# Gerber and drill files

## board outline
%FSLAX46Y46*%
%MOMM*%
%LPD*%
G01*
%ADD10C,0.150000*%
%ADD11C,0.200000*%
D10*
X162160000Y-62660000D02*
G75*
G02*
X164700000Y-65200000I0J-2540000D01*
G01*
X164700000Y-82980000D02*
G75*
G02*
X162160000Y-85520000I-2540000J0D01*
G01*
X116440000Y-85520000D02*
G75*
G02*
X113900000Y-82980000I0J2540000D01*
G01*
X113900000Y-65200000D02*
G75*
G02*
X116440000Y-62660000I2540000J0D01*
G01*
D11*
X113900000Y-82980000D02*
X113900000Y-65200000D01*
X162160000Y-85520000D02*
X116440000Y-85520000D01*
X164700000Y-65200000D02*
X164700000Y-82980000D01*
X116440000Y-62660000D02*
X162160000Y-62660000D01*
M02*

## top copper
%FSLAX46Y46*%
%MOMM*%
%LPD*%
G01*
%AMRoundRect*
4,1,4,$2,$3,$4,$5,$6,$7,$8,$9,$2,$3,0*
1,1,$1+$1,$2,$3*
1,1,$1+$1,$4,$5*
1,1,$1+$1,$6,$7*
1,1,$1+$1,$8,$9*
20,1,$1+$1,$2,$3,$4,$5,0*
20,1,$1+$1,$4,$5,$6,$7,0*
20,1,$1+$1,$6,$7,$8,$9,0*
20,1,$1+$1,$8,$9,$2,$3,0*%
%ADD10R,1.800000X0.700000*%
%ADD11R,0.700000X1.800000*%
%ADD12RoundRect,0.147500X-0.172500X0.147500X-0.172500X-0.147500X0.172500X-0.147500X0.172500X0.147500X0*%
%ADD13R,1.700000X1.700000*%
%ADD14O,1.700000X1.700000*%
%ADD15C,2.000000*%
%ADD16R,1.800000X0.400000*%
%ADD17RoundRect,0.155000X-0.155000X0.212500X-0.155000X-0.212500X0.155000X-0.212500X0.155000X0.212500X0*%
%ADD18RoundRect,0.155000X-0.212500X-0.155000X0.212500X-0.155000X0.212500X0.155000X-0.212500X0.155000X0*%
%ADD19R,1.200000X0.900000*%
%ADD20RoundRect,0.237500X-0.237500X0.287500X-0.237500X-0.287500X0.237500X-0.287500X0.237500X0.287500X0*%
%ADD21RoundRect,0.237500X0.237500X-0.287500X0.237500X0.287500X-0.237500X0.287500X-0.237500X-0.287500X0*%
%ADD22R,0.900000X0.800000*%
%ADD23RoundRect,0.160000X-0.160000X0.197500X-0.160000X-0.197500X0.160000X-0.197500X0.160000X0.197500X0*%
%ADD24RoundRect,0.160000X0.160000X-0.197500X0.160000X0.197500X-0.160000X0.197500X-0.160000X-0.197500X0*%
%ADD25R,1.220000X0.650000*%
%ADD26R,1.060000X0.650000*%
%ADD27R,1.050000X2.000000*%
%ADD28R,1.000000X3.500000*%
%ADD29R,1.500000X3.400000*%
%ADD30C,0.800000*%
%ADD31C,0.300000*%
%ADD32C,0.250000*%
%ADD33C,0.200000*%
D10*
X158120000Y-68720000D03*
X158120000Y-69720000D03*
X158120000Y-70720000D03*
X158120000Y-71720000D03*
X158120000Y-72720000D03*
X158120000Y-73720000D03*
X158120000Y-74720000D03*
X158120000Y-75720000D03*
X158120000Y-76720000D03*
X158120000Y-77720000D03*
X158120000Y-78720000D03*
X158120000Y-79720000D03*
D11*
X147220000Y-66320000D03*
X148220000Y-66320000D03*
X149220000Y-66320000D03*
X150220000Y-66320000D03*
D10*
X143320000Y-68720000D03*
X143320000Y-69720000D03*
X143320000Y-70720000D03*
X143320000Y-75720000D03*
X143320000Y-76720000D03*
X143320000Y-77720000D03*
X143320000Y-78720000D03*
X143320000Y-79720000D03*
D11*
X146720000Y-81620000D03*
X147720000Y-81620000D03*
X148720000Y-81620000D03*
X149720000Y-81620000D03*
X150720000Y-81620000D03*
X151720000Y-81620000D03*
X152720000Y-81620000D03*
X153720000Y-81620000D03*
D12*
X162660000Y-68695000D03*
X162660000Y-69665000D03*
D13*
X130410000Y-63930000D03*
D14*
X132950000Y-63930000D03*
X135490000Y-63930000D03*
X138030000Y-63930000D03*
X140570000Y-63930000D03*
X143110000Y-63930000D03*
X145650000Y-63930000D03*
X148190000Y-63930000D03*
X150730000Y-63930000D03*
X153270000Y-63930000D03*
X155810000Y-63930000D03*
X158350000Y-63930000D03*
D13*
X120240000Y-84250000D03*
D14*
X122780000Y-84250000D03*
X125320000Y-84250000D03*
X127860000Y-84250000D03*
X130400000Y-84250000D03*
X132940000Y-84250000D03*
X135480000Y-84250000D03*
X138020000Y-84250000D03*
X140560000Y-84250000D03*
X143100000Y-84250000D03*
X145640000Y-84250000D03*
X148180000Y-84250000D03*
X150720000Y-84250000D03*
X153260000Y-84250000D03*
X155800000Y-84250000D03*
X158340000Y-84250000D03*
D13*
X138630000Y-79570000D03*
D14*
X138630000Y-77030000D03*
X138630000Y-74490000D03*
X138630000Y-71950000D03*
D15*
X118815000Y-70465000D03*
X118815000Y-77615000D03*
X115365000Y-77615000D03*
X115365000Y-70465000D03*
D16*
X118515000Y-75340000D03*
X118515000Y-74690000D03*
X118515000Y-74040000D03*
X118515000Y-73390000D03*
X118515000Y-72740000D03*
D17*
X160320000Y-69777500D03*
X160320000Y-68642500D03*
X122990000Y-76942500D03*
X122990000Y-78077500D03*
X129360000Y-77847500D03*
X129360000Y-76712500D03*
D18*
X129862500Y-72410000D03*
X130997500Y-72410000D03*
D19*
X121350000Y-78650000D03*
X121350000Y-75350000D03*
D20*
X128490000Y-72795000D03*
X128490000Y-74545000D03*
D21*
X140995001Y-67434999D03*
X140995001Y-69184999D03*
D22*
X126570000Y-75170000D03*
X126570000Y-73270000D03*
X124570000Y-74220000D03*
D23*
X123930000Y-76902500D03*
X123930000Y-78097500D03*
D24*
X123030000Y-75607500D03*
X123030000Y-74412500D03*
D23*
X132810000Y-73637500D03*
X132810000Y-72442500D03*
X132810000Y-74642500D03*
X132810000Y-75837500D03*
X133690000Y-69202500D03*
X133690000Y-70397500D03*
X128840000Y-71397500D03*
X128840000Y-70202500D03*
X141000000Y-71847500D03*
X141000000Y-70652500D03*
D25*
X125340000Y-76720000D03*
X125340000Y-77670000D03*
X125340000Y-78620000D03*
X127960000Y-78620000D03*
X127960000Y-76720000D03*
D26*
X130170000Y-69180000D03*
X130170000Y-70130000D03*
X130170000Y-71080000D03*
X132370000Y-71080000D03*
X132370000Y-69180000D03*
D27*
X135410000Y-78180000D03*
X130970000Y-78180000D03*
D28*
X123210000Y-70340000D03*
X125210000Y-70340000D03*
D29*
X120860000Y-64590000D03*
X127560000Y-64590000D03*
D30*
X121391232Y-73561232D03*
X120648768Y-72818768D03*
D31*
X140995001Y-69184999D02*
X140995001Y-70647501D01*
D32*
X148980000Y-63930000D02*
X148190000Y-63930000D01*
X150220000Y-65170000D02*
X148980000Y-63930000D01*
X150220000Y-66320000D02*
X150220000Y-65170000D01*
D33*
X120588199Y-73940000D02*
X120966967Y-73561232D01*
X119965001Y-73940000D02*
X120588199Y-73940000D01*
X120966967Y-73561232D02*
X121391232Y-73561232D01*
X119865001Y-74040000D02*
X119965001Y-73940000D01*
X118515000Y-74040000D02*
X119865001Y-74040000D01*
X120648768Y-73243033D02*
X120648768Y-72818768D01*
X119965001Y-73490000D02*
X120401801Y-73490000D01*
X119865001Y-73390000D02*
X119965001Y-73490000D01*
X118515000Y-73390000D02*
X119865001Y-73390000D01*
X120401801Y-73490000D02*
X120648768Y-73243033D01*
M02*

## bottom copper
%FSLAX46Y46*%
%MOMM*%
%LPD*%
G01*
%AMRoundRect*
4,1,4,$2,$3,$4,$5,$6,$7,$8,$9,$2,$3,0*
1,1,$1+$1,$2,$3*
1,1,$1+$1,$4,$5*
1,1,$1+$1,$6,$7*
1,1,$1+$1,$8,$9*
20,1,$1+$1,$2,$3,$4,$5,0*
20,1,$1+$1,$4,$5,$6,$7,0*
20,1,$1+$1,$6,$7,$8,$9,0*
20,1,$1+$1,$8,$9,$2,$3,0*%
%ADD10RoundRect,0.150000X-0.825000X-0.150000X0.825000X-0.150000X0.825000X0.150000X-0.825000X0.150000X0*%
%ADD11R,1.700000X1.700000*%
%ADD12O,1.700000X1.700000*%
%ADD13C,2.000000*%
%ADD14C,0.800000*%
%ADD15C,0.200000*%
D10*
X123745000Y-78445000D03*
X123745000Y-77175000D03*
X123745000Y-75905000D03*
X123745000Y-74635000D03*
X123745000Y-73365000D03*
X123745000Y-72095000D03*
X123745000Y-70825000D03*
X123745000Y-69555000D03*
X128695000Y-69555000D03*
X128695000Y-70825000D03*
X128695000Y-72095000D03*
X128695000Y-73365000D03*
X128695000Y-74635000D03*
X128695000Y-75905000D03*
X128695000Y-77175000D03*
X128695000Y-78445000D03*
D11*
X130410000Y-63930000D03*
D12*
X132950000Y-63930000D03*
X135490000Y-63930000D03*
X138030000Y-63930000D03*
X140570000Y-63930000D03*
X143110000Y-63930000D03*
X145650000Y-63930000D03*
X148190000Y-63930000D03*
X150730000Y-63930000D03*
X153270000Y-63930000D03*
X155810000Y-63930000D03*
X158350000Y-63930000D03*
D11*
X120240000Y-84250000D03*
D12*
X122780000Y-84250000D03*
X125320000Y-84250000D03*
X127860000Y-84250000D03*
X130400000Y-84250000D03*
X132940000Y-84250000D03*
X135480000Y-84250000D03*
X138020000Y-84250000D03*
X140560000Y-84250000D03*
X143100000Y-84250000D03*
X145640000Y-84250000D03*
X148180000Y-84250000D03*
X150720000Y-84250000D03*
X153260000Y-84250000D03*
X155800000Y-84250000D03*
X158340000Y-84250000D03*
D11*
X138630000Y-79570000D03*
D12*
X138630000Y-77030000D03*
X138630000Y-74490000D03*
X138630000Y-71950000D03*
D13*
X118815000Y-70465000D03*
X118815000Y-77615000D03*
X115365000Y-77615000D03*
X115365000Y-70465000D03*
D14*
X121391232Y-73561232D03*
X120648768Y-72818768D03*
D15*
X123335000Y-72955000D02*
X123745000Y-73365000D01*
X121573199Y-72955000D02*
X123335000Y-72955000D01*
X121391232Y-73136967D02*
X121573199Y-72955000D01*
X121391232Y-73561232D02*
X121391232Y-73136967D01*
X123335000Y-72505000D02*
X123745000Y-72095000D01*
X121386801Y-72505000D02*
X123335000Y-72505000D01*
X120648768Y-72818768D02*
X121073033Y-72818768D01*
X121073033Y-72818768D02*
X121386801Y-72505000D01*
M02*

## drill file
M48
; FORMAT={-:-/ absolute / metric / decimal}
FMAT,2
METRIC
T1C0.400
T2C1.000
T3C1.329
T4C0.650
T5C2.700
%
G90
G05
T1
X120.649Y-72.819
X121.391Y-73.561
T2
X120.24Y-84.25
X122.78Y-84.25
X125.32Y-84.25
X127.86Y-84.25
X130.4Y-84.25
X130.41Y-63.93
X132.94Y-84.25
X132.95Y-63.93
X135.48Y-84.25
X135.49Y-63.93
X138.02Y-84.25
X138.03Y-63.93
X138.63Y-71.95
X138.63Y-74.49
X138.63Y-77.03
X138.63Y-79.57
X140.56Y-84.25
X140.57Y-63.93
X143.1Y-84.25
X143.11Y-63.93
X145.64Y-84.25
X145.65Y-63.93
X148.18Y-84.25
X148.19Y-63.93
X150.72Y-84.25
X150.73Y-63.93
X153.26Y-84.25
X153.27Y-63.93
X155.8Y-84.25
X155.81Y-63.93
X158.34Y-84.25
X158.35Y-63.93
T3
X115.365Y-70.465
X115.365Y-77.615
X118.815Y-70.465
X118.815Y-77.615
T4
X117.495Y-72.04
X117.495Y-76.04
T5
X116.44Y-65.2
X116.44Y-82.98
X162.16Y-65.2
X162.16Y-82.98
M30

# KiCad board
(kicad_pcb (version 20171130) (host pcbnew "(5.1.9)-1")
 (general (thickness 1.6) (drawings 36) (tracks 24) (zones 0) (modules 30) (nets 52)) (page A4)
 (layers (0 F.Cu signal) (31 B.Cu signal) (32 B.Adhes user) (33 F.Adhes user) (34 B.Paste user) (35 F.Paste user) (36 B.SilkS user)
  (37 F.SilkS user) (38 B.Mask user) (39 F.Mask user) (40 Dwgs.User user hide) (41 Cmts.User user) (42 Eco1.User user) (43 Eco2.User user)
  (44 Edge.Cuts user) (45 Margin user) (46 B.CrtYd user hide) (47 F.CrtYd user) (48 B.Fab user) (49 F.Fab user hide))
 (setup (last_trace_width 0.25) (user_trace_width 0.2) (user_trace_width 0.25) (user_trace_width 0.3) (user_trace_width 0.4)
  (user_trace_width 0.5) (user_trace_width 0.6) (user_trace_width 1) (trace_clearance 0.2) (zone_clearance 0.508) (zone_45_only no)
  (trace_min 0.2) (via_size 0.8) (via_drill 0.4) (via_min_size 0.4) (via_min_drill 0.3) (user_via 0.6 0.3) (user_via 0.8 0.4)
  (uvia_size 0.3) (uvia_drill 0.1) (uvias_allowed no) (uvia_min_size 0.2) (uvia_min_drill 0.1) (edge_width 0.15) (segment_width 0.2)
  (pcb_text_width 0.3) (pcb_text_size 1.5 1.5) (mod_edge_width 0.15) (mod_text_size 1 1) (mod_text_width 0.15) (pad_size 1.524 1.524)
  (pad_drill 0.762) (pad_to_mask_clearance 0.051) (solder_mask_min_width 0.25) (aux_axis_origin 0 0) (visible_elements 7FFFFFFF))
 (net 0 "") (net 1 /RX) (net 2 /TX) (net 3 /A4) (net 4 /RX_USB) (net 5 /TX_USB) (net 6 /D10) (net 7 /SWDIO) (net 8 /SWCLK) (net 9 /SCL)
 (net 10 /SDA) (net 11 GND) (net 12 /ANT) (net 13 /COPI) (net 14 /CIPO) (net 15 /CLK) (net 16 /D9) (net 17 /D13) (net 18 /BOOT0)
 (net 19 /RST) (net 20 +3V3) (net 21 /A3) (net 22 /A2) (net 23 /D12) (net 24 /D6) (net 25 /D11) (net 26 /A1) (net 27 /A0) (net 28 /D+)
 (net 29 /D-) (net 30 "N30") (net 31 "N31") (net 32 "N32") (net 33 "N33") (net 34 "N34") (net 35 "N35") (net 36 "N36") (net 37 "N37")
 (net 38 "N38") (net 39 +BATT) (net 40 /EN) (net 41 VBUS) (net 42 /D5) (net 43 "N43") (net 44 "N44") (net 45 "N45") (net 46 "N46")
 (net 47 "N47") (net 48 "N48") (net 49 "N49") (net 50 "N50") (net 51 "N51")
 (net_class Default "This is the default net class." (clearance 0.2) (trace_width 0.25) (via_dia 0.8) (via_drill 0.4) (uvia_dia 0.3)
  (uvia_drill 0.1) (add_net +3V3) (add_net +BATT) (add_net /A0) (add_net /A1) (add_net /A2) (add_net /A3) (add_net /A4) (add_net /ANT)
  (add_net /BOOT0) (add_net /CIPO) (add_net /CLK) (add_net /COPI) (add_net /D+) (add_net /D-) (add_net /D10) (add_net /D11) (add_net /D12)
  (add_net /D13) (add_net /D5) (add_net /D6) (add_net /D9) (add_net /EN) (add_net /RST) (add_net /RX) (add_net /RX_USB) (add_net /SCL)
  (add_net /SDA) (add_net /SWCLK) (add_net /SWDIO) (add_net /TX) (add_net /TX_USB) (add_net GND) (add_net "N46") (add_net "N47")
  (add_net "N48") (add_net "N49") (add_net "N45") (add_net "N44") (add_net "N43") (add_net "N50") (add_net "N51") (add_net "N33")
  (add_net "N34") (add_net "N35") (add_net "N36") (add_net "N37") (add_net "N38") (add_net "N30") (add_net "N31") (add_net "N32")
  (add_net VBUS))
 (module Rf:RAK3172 (layer F.Cu) (at 158.22 66.22 270)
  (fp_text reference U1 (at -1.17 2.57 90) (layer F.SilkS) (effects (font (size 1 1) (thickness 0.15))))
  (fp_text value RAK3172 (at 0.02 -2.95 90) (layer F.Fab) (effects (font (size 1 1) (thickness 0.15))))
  (pad 1 smd rect (at 2.5 0.1 270) (size 0.7 1.8) (layers F.Cu F.Paste F.Mask) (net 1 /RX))
  (pad 2 smd rect (at 3.5 0.1 270) (size 0.7 1.8) (layers F.Cu F.Paste F.Mask) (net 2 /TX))
  (pad 3 smd rect (at 4.5 0.1 270) (size 0.7 1.8) (layers F.Cu F.Paste F.Mask) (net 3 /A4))
  (pad 4 smd rect (at 5.5 0.1 270) (size 0.7 1.8) (layers F.Cu F.Paste F.Mask) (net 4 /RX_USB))
  (pad 5 smd rect (at 6.5 0.1 270) (size 0.7 1.8) (layers F.Cu F.Paste F.Mask) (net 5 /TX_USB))
  (pad 6 smd rect (at 7.5 0.1 270) (size 0.7 1.8) (layers F.Cu F.Paste F.Mask) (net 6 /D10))
  (pad 7 smd rect (at 8.5 0.1 270) (size 0.7 1.8) (layers F.Cu F.Paste F.Mask) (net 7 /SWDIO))
  (pad 8 smd rect (at 9.5 0.1 270) (size 0.7 1.8) (layers F.Cu F.Paste F.Mask) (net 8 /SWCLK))
  (pad 9 smd rect (at 10.5 0.1 270) (size 0.7 1.8) (layers F.Cu F.Paste F.Mask) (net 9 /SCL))
  (pad 10 smd rect (at 11.5 0.1 270) (size 0.7 1.8) (layers F.Cu F.Paste F.Mask) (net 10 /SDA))
  (pad 11 smd rect (at 12.5 0.1 270) (size 0.7 1.8) (layers F.Cu F.Paste F.Mask) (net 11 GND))
  (pad 12 smd rect (at 13.5 0.1 270) (size 0.7 1.8) (layers F.Cu F.Paste F.Mask) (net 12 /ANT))
  (pad 13 smd rect (at 0.1 11) (size 0.7 1.8) (layers F.Cu F.Paste F.Mask) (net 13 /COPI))
  (pad 14 smd rect (at 0.1 10) (size 0.7 1.8) (layers F.Cu F.Paste F.Mask) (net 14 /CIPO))
  (pad 15 smd rect (at 0.1 9) (size 0.7 1.8) (layers F.Cu F.Paste F.Mask) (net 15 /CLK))
  (pad 16 smd rect (at 0.1 8) (size 0.7 1.8) (layers F.Cu F.Paste F.Mask) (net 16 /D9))
  (pad 17 smd rect (at 2.5 14.9 270) (size 0.7 1.8) (layers F.Cu F.Paste F.Mask) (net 11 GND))
  (pad 18 smd rect (at 3.5 14.9 270) (size 0.7 1.8) (layers F.Cu F.Paste F.Mask) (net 11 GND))
  (pad 19 smd rect (at 4.5 14.9 270) (size 0.7 1.8) (layers F.Cu F.Paste F.Mask) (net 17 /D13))
  (pad 20 smd rect (at 9.5 14.9 270) (size 0.7 1.8) (layers F.Cu F.Paste F.Mask))
  (pad 21 smd rect (at 10.5 14.9 270) (size 0.7 1.8) (layers F.Cu F.Paste F.Mask) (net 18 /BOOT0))
  (pad 22 smd rect (at 11.5 14.9 270) (size 0.7 1.8) (layers F.Cu F.Paste F.Mask) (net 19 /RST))
  (pad 23 smd rect (at 12.5 14.9 270) (size 0.7 1.8) (layers F.Cu F.Paste F.Mask) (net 11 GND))
  (pad 24 smd rect (at 13.5 14.9 270) (size 0.7 1.8) (layers F.Cu F.Paste F.Mask) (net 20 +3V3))
  (pad 25 smd rect (at 15.4 11.5) (size 0.7 1.8) (layers F.Cu F.Paste F.Mask) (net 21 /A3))
  (pad 26 smd rect (at 15.4 10.5) (size 0.7 1.8) (layers F.Cu F.Paste F.Mask) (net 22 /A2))
  (pad 27 smd rect (at 15.4 9.5) (size 0.7 1.8) (layers F.Cu F.Paste F.Mask) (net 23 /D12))
  (pad 28 smd rect (at 15.4 8.5) (size 0.7 1.8) (layers F.Cu F.Paste F.Mask) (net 11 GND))
  (pad 29 smd rect (at 15.4 7.5) (size 0.7 1.8) (layers F.Cu F.Paste F.Mask) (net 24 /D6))
  (pad 30 smd rect (at 15.4 6.5) (size 0.7 1.8) (layers F.Cu F.Paste F.Mask) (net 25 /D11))
  (pad 31 smd rect (at 15.4 5.5) (size 0.7 1.8) (layers F.Cu F.Paste F.Mask) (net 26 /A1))
  (pad 32 smd rect (at 15.4 4.5) (size 0.7 1.8) (layers F.Cu F.Paste F.Mask) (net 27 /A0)))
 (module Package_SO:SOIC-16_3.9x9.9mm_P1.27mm (layer B.Cu) (at 126.22 74)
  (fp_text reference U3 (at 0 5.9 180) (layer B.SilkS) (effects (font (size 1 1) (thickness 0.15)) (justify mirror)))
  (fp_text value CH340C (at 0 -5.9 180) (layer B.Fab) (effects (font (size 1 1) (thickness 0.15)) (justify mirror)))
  (pad 1 smd roundrect (at -2.475 4.445) (size 1.95 0.6) (layers B.Cu B.Paste B.Mask) (roundrect_rratio 0.25) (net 11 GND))
  (pad 2 smd roundrect (at -2.475 3.175) (size 1.95 0.6) (layers B.Cu B.Paste B.Mask) (roundrect_rratio 0.25) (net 5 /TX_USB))
  (pad 3 smd roundrect (at -2.475 1.905) (size 1.95 0.6) (layers B.Cu B.Paste B.Mask) (roundrect_rratio 0.25) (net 4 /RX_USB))
  (pad 4 smd roundrect (at -2.475 0.635) (size 1.95 0.6) (layers B.Cu B.Paste B.Mask) (roundrect_rratio 0.25) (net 20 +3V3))
  (pad 5 smd roundrect (at -2.475 -0.635) (size 1.95 0.6) (layers B.Cu B.Paste B.Mask) (roundrect_rratio 0.25) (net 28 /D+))
  (pad 6 smd roundrect (at -2.475 -1.905) (size 1.95 0.6) (layers B.Cu B.Paste B.Mask) (roundrect_rratio 0.25) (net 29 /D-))
  (pad 7 smd roundrect (at -2.475 -3.175) (size 1.95 0.6) (layers B.Cu B.Paste B.Mask) (roundrect_rratio 0.25) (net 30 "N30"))
  (pad 8 smd roundrect (at -2.475 -4.445) (size 1.95 0.6) (layers B.Cu B.Paste B.Mask) (roundrect_rratio 0.25) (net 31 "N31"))
  (pad 9 smd roundrect (at 2.475 -4.445) (size 1.95 0.6) (layers B.Cu B.Paste B.Mask) (roundrect_rratio 0.25) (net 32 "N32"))
  (pad 10 smd roundrect (at 2.475 -3.175) (size 1.95 0.6) (layers B.Cu B.Paste B.Mask) (roundrect_rratio 0.25) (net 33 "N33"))
  (pad 11 smd roundrect (at 2.475 -1.905) (size 1.95 0.6) (layers B.Cu B.Paste B.Mask) (roundrect_rratio 0.25) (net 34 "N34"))
  (pad 12 smd roundrect (at 2.475 -0.635) (size 1.95 0.6) (layers B.Cu B.Paste B.Mask) (roundrect_rratio 0.25) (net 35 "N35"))
  (pad 13 smd roundrect (at 2.475 0.635) (size 1.95 0.6) (layers B.Cu B.Paste B.Mask) (roundrect_rratio 0.25) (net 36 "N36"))
  (pad 14 smd roundrect (at 2.475 1.905) (size 1.95 0.6) (layers B.Cu B.Paste B.Mask) (roundrect_rratio 0.25) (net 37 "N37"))
  (pad 15 smd roundrect (at 2.475 3.175) (size 1.95 0.6) (layers B.Cu B.Paste B.Mask) (roundrect_rratio 0.25) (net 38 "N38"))
  (pad 16 smd roundrect (at 2.475 4.445) (size 1.95 0.6) (layers B.Cu B.Paste B.Mask) (roundrect_rratio 0.25) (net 20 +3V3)))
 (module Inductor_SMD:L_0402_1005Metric (layer F.Cu) (at 162.66 69.18 270)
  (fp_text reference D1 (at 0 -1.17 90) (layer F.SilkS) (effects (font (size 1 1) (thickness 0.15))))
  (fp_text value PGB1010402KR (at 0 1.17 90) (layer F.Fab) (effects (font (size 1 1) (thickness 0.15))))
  (pad 1 smd roundrect (at -0.485 0 270) (size 0.59 0.64) (layers F.Cu F.Paste F.Mask) (roundrect_rratio 0.25) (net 12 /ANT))
  (pad 2 smd roundrect (at 0.485 0 270) (size 0.59 0.64) (layers F.Cu F.Paste F.Mask) (roundrect_rratio 0.25) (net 11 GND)))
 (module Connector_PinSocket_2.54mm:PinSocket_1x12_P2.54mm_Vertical (layer F.Cu) (at 130.41 63.93 90)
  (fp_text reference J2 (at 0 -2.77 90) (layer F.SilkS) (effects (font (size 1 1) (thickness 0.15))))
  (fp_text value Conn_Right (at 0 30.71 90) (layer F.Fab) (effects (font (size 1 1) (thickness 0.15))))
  (pad 1 thru_hole rect (at 0 0 90) (size 1.7 1.7) (drill 1) (layers *.Cu *.Mask) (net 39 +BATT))
  (pad 2 thru_hole oval (at 0 2.54 90) (size 1.7 1.7) (drill 1) (layers *.Cu *.Mask) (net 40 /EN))
  (pad 3 thru_hole oval (at 0 5.08 90) (size 1.7 1.7) (drill 1) (layers *.Cu *.Mask) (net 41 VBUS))
  (pad 4 thru_hole oval (at 0 7.62 90) (size 1.7 1.7) (drill 1) (layers *.Cu *.Mask) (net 17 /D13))
  (pad 5 thru_hole oval (at 0 10.16 90) (size 1.7 1.7) (drill 1) (layers *.Cu *.Mask) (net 23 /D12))
  (pad 6 thru_hole oval (at 0 12.7 90) (size 1.7 1.7) (drill 1) (layers *.Cu *.Mask) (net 25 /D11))
  (pad 7 thru_hole oval (at 0 15.24 90) (size 1.7 1.7) (drill 1) (layers *.Cu *.Mask) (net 6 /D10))
  (pad 8 thru_hole oval (at 0 17.78 90) (size 1.7 1.7) (drill 1) (layers *.Cu *.Mask) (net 16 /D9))
  (pad 9 thru_hole oval (at 0 20.32 90) (size 1.7 1.7) (drill 1) (layers *.Cu *.Mask) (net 24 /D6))
  (pad 10 thru_hole oval (at 0 22.86 90) (size 1.7 1.7) (drill 1) (layers *.Cu *.Mask) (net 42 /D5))
  (pad 11 thru_hole oval (at 0 25.4 90) (size 1.7 1.7) (drill 1) (layers *.Cu *.Mask) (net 9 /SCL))
  (pad 12 thru_hole oval (at 0 27.94 90) (size 1.7 1.7) (drill 1) (layers *.Cu *.Mask) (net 10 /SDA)))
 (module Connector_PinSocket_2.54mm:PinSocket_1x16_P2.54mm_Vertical (layer F.Cu) (at 120.24 84.25 90)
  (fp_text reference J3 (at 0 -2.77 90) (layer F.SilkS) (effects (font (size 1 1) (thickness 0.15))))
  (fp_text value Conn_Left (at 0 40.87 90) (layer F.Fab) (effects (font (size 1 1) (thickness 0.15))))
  (pad 1 thru_hole rect (at 0 0 90) (size 1.7 1.7) (drill 1) (layers *.Cu *.Mask) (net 19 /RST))
  (pad 2 thru_hole oval (at 0 2.54 90) (size 1.7 1.7) (drill 1) (layers *.Cu *.Mask) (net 20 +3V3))
  (pad 3 thru_hole oval (at 0 5.08 90) (size 1.7 1.7) (drill 1) (layers *.Cu *.Mask) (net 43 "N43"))
  (pad 4 thru_hole oval (at 0 7.62 90) (size 1.7 1.7) (drill 1) (layers *.Cu *.Mask) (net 11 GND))
  (pad 5 thru_hole oval (at 0 10.16 90) (size 1.7 1.7) (drill 1) (layers *.Cu *.Mask) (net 27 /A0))
  (pad 6 thru_hole oval (at 0 12.7 90) (size 1.7 1.7) (drill 1) (layers *.Cu *.Mask) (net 26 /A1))
  (pad 7 thru_hole oval (at 0 15.24 90) (size 1.7 1.7) (drill 1) (layers *.Cu *.Mask) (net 22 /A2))
  (pad 8 thru_hole oval (at 0 17.78 90) (size 1.7 1.7) (drill 1) (layers *.Cu *.Mask) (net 21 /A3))
  (pad 9 thru_hole oval (at 0 20.32 90) (size 1.7 1.7) (drill 1) (layers *.Cu *.Mask) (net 3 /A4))
  (pad 10 thru_hole oval (at 0 22.86 90) (size 1.7 1.7) (drill 1) (layers *.Cu *.Mask) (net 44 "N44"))
  (pad 11 thru_hole oval (at 0 25.4 90) (size 1.7 1.7) (drill 1) (layers *.Cu *.Mask) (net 15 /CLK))
  (pad 12 thru_hole oval (at 0 27.94 90) (size 1.7 1.7) (drill 1) (layers *.Cu *.Mask) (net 13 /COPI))
  (pad 13 thru_hole oval (at 0 30.48 90) (size 1.7 1.7) (drill 1) (layers *.Cu *.Mask) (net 14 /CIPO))
  (pad 14 thru_hole oval (at 0 33.02 90) (size 1.7 1.7) (drill 1) (layers *.Cu *.Mask) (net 1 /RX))
  (pad 15 thru_hole oval (at 0 35.56 90) (size 1.7 1.7) (drill 1) (layers *.Cu *.Mask) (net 2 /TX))
  (pad 16 thru_hole oval (at 0 38.1 90) (size 1.7 1.7) (drill 1) (layers *.Cu *.Mask) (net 18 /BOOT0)))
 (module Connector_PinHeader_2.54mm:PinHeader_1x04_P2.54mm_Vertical (layer F.Cu) (at 138.63 79.57 180)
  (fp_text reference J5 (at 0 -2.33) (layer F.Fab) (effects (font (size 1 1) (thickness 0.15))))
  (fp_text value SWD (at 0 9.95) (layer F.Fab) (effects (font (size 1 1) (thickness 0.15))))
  (pad 1 thru_hole rect (at 0 0 180) (size 1.7 1.7) (drill 1) (layers *.Cu *.Mask) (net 20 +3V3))
  (pad 2 thru_hole oval (at 0 2.54 180) (size 1.7 1.7) (drill 1) (layers *.Cu *.Mask) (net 7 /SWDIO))
  (pad 3 thru_hole oval (at 0 5.08 180) (size 1.7 1.7) (drill 1) (layers *.Cu *.Mask) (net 8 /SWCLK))
  (pad 4 thru_hole oval (at 0 7.62 180) (size 1.7 1.7) (drill 1) (layers *.Cu *.Mask) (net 11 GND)))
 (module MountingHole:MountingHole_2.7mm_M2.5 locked (layer F.Cu) (at 162.16 65.2)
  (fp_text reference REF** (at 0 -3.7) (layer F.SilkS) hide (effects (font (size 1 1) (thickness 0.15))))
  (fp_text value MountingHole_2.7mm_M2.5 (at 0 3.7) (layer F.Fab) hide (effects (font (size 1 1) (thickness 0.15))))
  (pad 1 np_thru_hole circle (at 0 0) (size 2.7 2.7) (drill 2.7) (layers *.Cu *.Mask)))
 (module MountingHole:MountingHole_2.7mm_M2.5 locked (layer F.Cu) (at 162.16 82.98)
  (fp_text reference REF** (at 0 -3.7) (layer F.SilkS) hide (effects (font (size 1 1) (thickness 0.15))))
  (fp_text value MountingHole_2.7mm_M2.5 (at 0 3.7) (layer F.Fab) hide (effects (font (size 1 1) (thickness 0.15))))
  (pad 1 np_thru_hole circle (at 0 0) (size 2.7 2.7) (drill 2.7) (layers *.Cu *.Mask)))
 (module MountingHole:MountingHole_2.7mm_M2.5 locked (layer F.Cu) (at 116.44 82.98)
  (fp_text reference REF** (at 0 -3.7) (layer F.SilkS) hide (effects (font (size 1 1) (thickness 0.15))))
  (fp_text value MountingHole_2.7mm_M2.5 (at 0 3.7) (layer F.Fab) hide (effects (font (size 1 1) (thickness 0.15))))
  (pad 1 np_thru_hole circle (at 0 0) (size 2.7 2.7) (drill 2.7) (layers *.Cu *.Mask)))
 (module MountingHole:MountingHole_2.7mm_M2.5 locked (layer F.Cu) (at 116.44 65.2)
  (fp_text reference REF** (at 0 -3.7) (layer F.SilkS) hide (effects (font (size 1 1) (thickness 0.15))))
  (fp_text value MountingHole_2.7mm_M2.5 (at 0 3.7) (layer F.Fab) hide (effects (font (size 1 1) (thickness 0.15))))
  (pad 1 np_thru_hole circle (at 0 0) (size 2.7 2.7) (drill 2.7) (layers *.Cu *.Mask)))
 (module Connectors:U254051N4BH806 (layer F.Cu) (at 116.33 74.04 270)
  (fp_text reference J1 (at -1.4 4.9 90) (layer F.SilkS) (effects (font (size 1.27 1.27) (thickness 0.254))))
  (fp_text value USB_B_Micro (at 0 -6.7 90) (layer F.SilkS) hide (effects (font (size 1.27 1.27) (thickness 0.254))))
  (pad MH6 np_thru_hole circle (at 2 -1.165 270) (size 0.65 0) (drill 0.65) (layers *.Cu *.Mask))
  (pad MH5 np_thru_hole circle (at -2 -1.165 270) (size 0.65 0) (drill 0.65) (layers *.Cu *.Mask))
  (pad 6 thru_hole circle (at -3.575 -2.485 270) (size 2 2) (drill 1.3285) (layers *.Cu *.Mask) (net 11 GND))
  (pad 6 thru_hole circle (at 3.575 -2.485 270) (size 2 2) (drill 1.3285) (layers *.Cu *.Mask) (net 11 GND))
  (pad 6 thru_hole circle (at 3.575 0.965 270) (size 2 2) (drill 1.3285) (layers *.Cu *.Mask) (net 11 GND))
  (pad 6 thru_hole circle (at -3.575 0.965 270) (size 2 2) (drill 1.3285) (layers *.Cu *.Mask) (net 11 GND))
  (pad 5 smd rect (at 1.3 -2.185 270) (size 0.4 1.8) (layers F.Cu F.Paste F.Mask) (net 11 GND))
  (pad 4 smd rect (at 0.65 -2.185 270) (size 0.4 1.8) (layers F.Cu F.Paste F.Mask) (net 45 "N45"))
  (pad 3 smd rect (at 0 -2.185 270) (size 0.4 1.8) (layers F.Cu F.Paste F.Mask) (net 28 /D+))
  (pad 2 smd rect (at -0.65 -2.185 270) (size 0.4 1.8) (layers F.Cu F.Paste F.Mask) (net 29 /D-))
  (pad 1 smd rect (at -1.3 -2.185 270) (size 0.4 1.8) (layers F.Cu F.Paste F.Mask) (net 41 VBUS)))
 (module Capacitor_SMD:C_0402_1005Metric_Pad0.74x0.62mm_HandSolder (layer F.Cu) (at 160.32 69.21 270)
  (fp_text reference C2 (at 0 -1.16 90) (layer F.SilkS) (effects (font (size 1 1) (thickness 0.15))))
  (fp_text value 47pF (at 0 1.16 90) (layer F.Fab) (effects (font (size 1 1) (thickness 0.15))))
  (pad 2 smd roundrect (at 0.5675 0 270) (size 0.735 0.62) (layers F.Cu F.Paste F.Mask) (roundrect_rratio 0.25) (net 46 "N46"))
  (pad 1 smd roundrect (at -0.5675 0 270) (size 0.735 0.62) (layers F.Cu F.Paste F.Mask) (roundrect_rratio 0.25) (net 12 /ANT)))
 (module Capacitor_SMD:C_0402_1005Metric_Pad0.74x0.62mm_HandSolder (layer F.Cu) (at 122.99 77.51 270)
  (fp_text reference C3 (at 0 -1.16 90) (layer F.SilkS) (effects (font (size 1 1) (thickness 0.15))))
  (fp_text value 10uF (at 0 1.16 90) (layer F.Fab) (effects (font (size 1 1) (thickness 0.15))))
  (pad 1 smd roundrect (at -0.5675 0 270) (size 0.735 0.62) (layers F.Cu F.Paste F.Mask) (roundrect_rratio 0.25) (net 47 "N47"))
  (pad 2 smd roundrect (at 0.5675 0 270) (size 0.735 0.62) (layers F.Cu F.Paste F.Mask) (roundrect_rratio 0.25) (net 11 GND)))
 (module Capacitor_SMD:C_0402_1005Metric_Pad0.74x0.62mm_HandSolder (layer F.Cu) (at 129.36 77.28 270)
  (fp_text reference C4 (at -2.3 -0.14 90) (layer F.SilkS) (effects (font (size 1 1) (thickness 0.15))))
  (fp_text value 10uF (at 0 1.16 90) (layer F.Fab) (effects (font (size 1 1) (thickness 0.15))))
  (pad 2 smd roundrect (at 0.5675 0 270) (size 0.735 0.62) (layers F.Cu F.Paste F.Mask) (roundrect_rratio 0.25) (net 11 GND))
  (pad 1 smd roundrect (at -0.5675 0 270) (size 0.735 0.62) (layers F.Cu F.Paste F.Mask) (roundrect_rratio 0.25) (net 20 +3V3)))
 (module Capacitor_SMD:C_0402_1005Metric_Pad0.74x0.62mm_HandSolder (layer F.Cu) (at 130.43 72.41)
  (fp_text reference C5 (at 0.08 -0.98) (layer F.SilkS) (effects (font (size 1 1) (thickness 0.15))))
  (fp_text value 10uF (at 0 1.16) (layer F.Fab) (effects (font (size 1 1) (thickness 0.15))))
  (pad 1 smd roundrect (at -0.5675 0) (size 0.735 0.62) (layers F.Cu F.Paste F.Mask) (roundrect_rratio 0.25) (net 39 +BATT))
  (pad 2 smd roundrect (at 0.5675 0) (size 0.735 0.62) (layers F.Cu F.Paste F.Mask) (roundrect_rratio 0.25) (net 11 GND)))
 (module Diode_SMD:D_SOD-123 (layer F.Cu) (at 121.35 77 90)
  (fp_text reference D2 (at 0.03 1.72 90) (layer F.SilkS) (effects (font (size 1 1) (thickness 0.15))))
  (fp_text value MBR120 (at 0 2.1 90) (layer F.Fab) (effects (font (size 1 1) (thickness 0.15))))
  (pad 1 smd rect (at -1.65 0 90) (size 0.9 1.2) (layers F.Cu F.Paste F.Mask) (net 47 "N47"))
  (pad 2 smd rect (at 1.65 0 90) (size 0.9 1.2) (layers F.Cu F.Paste F.Mask) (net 41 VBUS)))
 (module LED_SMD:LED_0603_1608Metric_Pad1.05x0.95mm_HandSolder (layer F.Cu) (at 128.49 73.67 270)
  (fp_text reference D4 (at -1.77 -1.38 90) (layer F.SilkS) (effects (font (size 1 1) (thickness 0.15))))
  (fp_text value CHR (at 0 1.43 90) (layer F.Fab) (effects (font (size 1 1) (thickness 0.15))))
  (pad 1 smd roundrect (at -0.875 0 270) (size 1.05 0.95) (layers F.Cu F.Paste F.Mask) (roundrect_rratio 0.25) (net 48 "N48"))
  (pad 2 smd roundrect (at 0.875 0 270) (size 1.05 0.95) (layers F.Cu F.Paste F.Mask) (roundrect_rratio 0.25) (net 41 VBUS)))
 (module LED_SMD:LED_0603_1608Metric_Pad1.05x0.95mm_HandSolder (layer F.Cu) (at 140.995001 68.309999 90)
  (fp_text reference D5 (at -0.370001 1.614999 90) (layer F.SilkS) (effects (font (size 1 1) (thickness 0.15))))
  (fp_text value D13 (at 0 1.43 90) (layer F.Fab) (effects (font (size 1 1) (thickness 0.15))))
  (pad 2 smd roundrect (at 0.875 0 90) (size 1.05 0.95) (layers F.Cu F.Paste F.Mask) (roundrect_rratio 0.25) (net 17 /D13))
  (pad 1 smd roundrect (at -0.875 0 90) (size 1.05 0.95) (layers F.Cu F.Paste F.Mask) (roundrect_rratio 0.25) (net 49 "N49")))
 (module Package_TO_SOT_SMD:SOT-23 (layer F.Cu) (at 125.57 74.22 180)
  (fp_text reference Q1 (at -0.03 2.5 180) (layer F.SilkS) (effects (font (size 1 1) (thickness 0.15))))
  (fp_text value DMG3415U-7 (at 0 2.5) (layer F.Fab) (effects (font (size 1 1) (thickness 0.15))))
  (pad 1 smd rect (at -1 -0.95 180) (size 0.9 0.8) (layers F.Cu F.Paste F.Mask) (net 41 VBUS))
  (pad 2 smd rect (at -1 0.95 180) (size 0.9 0.8) (layers F.Cu F.Paste F.Mask) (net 47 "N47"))
  (pad 3 smd rect (at 1 0 180) (size 0.9 0.8) (layers F.Cu F.Paste F.Mask) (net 39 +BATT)))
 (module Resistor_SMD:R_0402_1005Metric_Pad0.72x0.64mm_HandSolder (layer F.Cu) (at 123.93 77.5 270)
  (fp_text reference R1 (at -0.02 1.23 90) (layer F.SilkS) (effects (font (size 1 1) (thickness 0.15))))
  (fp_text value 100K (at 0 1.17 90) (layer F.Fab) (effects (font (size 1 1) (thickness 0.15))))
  (pad 1 smd roundrect (at -0.5975 0 270) (size 0.715 0.64) (layers F.Cu F.Paste F.Mask) (roundrect_rratio 0.25) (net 47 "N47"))
  (pad 2 smd roundrect (at 0.5975 0 270) (size 0.715 0.64) (layers F.Cu F.Paste F.Mask) (roundrect_rratio 0.25) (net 40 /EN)))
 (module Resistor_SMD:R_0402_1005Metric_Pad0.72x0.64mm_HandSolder (layer F.Cu) (at 123.03 75.01 90)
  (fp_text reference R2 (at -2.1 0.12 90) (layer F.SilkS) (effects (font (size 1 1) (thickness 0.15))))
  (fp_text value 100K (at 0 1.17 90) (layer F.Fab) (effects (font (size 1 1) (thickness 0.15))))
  (pad 1 smd roundrect (at -0.5975 0 90) (size 0.715 0.64) (layers F.Cu F.Paste F.Mask) (roundrect_rratio 0.25) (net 41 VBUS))
  (pad 2 smd roundrect (at 0.5975 0 90) (size 0.715 0.64) (layers F.Cu F.Paste F.Mask) (roundrect_rratio 0.25) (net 11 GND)))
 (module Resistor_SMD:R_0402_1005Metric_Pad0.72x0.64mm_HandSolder (layer F.Cu) (at 132.81 73.04 270)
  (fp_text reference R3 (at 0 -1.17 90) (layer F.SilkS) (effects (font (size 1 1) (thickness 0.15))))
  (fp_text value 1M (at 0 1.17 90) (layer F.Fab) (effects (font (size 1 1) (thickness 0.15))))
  (pad 2 smd roundrect (at 0.5975 0 270) (size 0.715 0.64) (layers F.Cu F.Paste F.Mask) (roundrect_rratio 0.25) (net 27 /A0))
  (pad 1 smd roundrect (at -0.5975 0 270) (size 0.715 0.64) (layers F.Cu F.Paste F.Mask) (roundrect_rratio 0.25) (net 39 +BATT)))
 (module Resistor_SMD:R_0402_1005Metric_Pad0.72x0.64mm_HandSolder (layer F.Cu) (at 132.81 75.24 270)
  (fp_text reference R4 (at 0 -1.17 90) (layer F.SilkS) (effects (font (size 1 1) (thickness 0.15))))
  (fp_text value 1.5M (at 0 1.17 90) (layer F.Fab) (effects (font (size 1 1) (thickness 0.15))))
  (pad 1 smd roundrect (at -0.5975 0 270) (size 0.715 0.64) (layers F.Cu F.Paste F.Mask) (roundrect_rratio 0.25) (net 27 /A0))
  (pad 2 smd roundrect (at 0.5975 0 270) (size 0.715 0.64) (layers F.Cu F.Paste F.Mask) (roundrect_rratio 0.25) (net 11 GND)))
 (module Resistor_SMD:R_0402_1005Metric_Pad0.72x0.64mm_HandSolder (layer F.Cu) (at 133.69 69.8 270)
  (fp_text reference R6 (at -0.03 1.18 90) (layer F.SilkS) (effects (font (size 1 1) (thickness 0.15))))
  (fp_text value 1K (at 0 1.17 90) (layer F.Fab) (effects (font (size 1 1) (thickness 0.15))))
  (pad 1 smd roundrect (at -0.5975 0 270) (size 0.715 0.64) (layers F.Cu F.Paste F.Mask) (roundrect_rratio 0.25) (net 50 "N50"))
  (pad 2 smd roundrect (at 0.5975 0 270) (size 0.715 0.64) (layers F.Cu F.Paste F.Mask) (roundrect_rratio 0.25) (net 11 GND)))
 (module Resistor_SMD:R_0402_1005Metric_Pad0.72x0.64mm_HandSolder (layer F.Cu) (at 128.84 70.8 270)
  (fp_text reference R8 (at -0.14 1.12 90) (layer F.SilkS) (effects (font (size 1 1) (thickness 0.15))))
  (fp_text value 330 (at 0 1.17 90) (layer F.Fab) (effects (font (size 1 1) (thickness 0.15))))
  (pad 2 smd roundrect (at 0.5975 0 270) (size 0.715 0.64) (layers F.Cu F.Paste F.Mask) (roundrect_rratio 0.25) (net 48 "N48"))
  (pad 1 smd roundrect (at -0.5975 0 270) (size 0.715 0.64) (layers F.Cu F.Paste F.Mask) (roundrect_rratio 0.25) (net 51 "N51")))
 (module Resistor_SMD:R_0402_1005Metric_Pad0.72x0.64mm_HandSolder (layer F.Cu) (at 141 71.25 270)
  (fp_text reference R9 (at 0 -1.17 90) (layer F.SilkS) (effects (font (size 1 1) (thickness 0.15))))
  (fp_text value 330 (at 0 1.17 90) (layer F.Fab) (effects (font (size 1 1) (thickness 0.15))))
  (pad 2 smd roundrect (at 0.5975 0 270) (size 0.715 0.64) (layers F.Cu F.Paste F.Mask) (roundrect_rratio 0.25) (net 11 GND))
  (pad 1 smd roundrect (at -0.5975 0 270) (size 0.715 0.64) (layers F.Cu F.Paste F.Mask) (roundrect_rratio 0.25) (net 49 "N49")))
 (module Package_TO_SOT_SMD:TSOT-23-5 (layer F.Cu) (at 126.65 77.67)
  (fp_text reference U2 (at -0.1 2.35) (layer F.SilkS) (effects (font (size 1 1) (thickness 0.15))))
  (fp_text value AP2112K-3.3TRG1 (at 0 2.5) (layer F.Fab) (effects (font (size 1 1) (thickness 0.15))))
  (pad 1 smd rect (at -1.31 -0.95) (size 1.22 0.65) (layers F.Cu F.Paste F.Mask) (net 47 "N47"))
  (pad 2 smd rect (at -1.31 0) (size 1.22 0.65) (layers F.Cu F.Paste F.Mask) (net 11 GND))
  (pad 3 smd rect (at -1.31 0.95) (size 1.22 0.65) (layers F.Cu F.Paste F.Mask) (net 40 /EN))
  (pad 4 smd rect (at 1.31 0.95) (size 1.22 0.65) (layers F.Cu F.Paste F.Mask))
  (pad 5 smd rect (at 1.31 -0.95) (size 1.22 0.65) (layers F.Cu F.Paste F.Mask) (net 20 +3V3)))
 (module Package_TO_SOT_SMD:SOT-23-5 (layer F.Cu) (at 131.27 70.13)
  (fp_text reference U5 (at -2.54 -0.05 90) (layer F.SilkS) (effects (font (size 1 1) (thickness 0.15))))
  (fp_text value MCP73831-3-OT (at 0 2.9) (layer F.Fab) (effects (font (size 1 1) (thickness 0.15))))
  (pad 1 smd rect (at -1.1 -0.95) (size 1.06 0.65) (layers F.Cu F.Paste F.Mask) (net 51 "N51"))
  (pad 2 smd rect (at -1.1 0) (size 1.06 0.65) (layers F.Cu F.Paste F.Mask) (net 11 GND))
  (pad 3 smd rect (at -1.1 0.95) (size 1.06 0.65) (layers F.Cu F.Paste F.Mask) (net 39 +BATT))
  (pad 4 smd rect (at 1.1 0.95) (size 1.06 0.65) (layers F.Cu F.Paste F.Mask) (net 41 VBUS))
  (pad 5 smd rect (at 1.1 -0.95) (size 1.06 0.65) (layers F.Cu F.Paste F.Mask) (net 50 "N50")))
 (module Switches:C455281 (layer F.Cu) (at 130.43 76.78)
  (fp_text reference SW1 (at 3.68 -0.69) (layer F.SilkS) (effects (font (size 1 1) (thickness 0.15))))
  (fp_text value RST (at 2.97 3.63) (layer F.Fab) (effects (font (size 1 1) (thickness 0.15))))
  (pad 1 smd rect (at 4.98 1.4) (size 1.05 2) (layers F.Cu F.Paste F.Mask) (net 11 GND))
  (pad 2 smd rect (at 0.54 1.4) (size 1.05 2) (layers F.Cu F.Paste F.Mask) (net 19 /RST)))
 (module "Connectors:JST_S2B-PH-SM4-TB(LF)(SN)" (layer F.Cu) (at 124.21 70.34 180)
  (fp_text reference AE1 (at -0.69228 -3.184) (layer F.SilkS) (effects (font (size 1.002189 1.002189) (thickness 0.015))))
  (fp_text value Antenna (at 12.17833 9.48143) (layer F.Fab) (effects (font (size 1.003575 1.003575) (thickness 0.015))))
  (pad 2 smd rect (at 1 0 180) (size 1 3.5) (layers F.Cu F.Paste F.Mask) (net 11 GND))
  (pad 1 smd rect (at -1 0 180) (size 1 3.5) (layers F.Cu F.Paste F.Mask) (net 46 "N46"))
  (pad S2 smd rect (at 3.35 5.75 180) (size 1.5 3.4) (layers F.Cu F.Paste F.Mask))
  (pad S1 smd rect (at -3.35 5.75 180) (size 1.5 3.4) (layers F.Cu F.Paste F.Mask)))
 (gr_arc (start 162.16 65.2) (end 164.7 65.2) (angle -90) (layer Edge.Cuts) (width 0.15))
 (gr_arc (start 162.16 82.98) (end 162.16 85.52) (angle -90) (layer Edge.Cuts) (width 0.15))
 (gr_arc (start 116.44 82.98) (end 113.9 82.98) (angle -90) (layer Edge.Cuts) (width 0.15))
 (gr_arc (start 116.44 65.2) (end 116.44 62.66) (angle -90) (layer Edge.Cuts) (width 0.15))
 (gr_line (start 113.9 82.98) (end 113.9 65.2) (layer Edge.Cuts) (width 0.2))
 (gr_line (start 162.16 85.52) (end 116.44 85.52) (layer Edge.Cuts) (width 0.2))
 (gr_line (start 164.7 65.2) (end 164.7 82.98) (layer Edge.Cuts) (width 0.2))
 (gr_line (start 116.44 62.66) (end 162.16 62.66) (layer Edge.Cuts) (width 0.2))
 (segment (start 140.995001 69.184999) (end 140.995001 70.647501) (width 0.3) (layer F.Cu) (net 49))
 (segment (start 148.98 63.93) (end 148.19 63.93) (width 0.25) (layer F.Cu) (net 16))
 (segment (start 150.22 65.17) (end 148.98 63.93) (width 0.25) (layer F.Cu) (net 16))
 (segment (start 150.22 66.32) (end 150.22 65.17) (width 0.25) (layer F.Cu) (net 16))
 (segment (start 120.588199 73.94) (end 120.966967 73.561232) (width 0.2) (layer F.Cu) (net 28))
 (segment (start 119.965001 73.94) (end 120.588199 73.94) (width 0.2) (layer F.Cu) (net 28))
 (segment (start 120.966967 73.561232) (end 121.391232 73.561232) (width 0.2) (layer F.Cu) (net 28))
 (segment (start 119.865001 74.04) (end 119.965001 73.94) (width 0.2) (layer F.Cu) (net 28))
 (segment (start 118.515 74.04) (end 119.865001 74.04) (width 0.2) (layer F.Cu) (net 28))
 (via (at 121.391232 73.561232) (size 0.8) (drill 0.4) (layers F.Cu B.Cu) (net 28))
 (segment (start 123.335 72.955) (end 123.745 73.365) (width 0.2) (layer B.Cu) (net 28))
 (segment (start 121.573199 72.955) (end 123.335 72.955) (width 0.2) (layer B.Cu) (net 28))
 (segment (start 121.391232 73.136967) (end 121.573199 72.955) (width 0.2) (layer B.Cu) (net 28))
 (segment (start 121.391232 73.561232) (end 121.391232 73.136967) (width 0.2) (layer B.Cu) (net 28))
 (segment (start 120.648768 73.243033) (end 120.648768 72.818768) (width 0.2) (layer F.Cu) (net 29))
 (segment (start 119.965001 73.49) (end 120.401801 73.49) (width 0.2) (layer F.Cu) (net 29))
 (segment (start 119.865001 73.39) (end 119.965001 73.49) (width 0.2) (layer F.Cu) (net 29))
 (segment (start 118.515 73.39) (end 119.865001 73.39) (width 0.2) (layer F.Cu) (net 29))
 (segment (start 120.401801 73.49) (end 120.648768 73.243033) (width 0.2) (layer F.Cu) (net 29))
 (via (at 120.648768 72.818768) (size 0.8) (drill 0.4) (layers F.Cu B.Cu) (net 29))
 (segment (start 123.335 72.505) (end 123.745 72.095) (width 0.2) (layer B.Cu) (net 29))
 (segment (start 121.386801 72.505) (end 123.335 72.505) (width 0.2) (layer B.Cu) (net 29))
 (segment (start 120.648768 72.818768) (end 121.073033 72.818768) (width 0.2) (layer B.Cu) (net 29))
 (segment (start 121.073033 72.818768) (end 121.386801 72.505) (width 0.2) (layer B.Cu) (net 29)))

